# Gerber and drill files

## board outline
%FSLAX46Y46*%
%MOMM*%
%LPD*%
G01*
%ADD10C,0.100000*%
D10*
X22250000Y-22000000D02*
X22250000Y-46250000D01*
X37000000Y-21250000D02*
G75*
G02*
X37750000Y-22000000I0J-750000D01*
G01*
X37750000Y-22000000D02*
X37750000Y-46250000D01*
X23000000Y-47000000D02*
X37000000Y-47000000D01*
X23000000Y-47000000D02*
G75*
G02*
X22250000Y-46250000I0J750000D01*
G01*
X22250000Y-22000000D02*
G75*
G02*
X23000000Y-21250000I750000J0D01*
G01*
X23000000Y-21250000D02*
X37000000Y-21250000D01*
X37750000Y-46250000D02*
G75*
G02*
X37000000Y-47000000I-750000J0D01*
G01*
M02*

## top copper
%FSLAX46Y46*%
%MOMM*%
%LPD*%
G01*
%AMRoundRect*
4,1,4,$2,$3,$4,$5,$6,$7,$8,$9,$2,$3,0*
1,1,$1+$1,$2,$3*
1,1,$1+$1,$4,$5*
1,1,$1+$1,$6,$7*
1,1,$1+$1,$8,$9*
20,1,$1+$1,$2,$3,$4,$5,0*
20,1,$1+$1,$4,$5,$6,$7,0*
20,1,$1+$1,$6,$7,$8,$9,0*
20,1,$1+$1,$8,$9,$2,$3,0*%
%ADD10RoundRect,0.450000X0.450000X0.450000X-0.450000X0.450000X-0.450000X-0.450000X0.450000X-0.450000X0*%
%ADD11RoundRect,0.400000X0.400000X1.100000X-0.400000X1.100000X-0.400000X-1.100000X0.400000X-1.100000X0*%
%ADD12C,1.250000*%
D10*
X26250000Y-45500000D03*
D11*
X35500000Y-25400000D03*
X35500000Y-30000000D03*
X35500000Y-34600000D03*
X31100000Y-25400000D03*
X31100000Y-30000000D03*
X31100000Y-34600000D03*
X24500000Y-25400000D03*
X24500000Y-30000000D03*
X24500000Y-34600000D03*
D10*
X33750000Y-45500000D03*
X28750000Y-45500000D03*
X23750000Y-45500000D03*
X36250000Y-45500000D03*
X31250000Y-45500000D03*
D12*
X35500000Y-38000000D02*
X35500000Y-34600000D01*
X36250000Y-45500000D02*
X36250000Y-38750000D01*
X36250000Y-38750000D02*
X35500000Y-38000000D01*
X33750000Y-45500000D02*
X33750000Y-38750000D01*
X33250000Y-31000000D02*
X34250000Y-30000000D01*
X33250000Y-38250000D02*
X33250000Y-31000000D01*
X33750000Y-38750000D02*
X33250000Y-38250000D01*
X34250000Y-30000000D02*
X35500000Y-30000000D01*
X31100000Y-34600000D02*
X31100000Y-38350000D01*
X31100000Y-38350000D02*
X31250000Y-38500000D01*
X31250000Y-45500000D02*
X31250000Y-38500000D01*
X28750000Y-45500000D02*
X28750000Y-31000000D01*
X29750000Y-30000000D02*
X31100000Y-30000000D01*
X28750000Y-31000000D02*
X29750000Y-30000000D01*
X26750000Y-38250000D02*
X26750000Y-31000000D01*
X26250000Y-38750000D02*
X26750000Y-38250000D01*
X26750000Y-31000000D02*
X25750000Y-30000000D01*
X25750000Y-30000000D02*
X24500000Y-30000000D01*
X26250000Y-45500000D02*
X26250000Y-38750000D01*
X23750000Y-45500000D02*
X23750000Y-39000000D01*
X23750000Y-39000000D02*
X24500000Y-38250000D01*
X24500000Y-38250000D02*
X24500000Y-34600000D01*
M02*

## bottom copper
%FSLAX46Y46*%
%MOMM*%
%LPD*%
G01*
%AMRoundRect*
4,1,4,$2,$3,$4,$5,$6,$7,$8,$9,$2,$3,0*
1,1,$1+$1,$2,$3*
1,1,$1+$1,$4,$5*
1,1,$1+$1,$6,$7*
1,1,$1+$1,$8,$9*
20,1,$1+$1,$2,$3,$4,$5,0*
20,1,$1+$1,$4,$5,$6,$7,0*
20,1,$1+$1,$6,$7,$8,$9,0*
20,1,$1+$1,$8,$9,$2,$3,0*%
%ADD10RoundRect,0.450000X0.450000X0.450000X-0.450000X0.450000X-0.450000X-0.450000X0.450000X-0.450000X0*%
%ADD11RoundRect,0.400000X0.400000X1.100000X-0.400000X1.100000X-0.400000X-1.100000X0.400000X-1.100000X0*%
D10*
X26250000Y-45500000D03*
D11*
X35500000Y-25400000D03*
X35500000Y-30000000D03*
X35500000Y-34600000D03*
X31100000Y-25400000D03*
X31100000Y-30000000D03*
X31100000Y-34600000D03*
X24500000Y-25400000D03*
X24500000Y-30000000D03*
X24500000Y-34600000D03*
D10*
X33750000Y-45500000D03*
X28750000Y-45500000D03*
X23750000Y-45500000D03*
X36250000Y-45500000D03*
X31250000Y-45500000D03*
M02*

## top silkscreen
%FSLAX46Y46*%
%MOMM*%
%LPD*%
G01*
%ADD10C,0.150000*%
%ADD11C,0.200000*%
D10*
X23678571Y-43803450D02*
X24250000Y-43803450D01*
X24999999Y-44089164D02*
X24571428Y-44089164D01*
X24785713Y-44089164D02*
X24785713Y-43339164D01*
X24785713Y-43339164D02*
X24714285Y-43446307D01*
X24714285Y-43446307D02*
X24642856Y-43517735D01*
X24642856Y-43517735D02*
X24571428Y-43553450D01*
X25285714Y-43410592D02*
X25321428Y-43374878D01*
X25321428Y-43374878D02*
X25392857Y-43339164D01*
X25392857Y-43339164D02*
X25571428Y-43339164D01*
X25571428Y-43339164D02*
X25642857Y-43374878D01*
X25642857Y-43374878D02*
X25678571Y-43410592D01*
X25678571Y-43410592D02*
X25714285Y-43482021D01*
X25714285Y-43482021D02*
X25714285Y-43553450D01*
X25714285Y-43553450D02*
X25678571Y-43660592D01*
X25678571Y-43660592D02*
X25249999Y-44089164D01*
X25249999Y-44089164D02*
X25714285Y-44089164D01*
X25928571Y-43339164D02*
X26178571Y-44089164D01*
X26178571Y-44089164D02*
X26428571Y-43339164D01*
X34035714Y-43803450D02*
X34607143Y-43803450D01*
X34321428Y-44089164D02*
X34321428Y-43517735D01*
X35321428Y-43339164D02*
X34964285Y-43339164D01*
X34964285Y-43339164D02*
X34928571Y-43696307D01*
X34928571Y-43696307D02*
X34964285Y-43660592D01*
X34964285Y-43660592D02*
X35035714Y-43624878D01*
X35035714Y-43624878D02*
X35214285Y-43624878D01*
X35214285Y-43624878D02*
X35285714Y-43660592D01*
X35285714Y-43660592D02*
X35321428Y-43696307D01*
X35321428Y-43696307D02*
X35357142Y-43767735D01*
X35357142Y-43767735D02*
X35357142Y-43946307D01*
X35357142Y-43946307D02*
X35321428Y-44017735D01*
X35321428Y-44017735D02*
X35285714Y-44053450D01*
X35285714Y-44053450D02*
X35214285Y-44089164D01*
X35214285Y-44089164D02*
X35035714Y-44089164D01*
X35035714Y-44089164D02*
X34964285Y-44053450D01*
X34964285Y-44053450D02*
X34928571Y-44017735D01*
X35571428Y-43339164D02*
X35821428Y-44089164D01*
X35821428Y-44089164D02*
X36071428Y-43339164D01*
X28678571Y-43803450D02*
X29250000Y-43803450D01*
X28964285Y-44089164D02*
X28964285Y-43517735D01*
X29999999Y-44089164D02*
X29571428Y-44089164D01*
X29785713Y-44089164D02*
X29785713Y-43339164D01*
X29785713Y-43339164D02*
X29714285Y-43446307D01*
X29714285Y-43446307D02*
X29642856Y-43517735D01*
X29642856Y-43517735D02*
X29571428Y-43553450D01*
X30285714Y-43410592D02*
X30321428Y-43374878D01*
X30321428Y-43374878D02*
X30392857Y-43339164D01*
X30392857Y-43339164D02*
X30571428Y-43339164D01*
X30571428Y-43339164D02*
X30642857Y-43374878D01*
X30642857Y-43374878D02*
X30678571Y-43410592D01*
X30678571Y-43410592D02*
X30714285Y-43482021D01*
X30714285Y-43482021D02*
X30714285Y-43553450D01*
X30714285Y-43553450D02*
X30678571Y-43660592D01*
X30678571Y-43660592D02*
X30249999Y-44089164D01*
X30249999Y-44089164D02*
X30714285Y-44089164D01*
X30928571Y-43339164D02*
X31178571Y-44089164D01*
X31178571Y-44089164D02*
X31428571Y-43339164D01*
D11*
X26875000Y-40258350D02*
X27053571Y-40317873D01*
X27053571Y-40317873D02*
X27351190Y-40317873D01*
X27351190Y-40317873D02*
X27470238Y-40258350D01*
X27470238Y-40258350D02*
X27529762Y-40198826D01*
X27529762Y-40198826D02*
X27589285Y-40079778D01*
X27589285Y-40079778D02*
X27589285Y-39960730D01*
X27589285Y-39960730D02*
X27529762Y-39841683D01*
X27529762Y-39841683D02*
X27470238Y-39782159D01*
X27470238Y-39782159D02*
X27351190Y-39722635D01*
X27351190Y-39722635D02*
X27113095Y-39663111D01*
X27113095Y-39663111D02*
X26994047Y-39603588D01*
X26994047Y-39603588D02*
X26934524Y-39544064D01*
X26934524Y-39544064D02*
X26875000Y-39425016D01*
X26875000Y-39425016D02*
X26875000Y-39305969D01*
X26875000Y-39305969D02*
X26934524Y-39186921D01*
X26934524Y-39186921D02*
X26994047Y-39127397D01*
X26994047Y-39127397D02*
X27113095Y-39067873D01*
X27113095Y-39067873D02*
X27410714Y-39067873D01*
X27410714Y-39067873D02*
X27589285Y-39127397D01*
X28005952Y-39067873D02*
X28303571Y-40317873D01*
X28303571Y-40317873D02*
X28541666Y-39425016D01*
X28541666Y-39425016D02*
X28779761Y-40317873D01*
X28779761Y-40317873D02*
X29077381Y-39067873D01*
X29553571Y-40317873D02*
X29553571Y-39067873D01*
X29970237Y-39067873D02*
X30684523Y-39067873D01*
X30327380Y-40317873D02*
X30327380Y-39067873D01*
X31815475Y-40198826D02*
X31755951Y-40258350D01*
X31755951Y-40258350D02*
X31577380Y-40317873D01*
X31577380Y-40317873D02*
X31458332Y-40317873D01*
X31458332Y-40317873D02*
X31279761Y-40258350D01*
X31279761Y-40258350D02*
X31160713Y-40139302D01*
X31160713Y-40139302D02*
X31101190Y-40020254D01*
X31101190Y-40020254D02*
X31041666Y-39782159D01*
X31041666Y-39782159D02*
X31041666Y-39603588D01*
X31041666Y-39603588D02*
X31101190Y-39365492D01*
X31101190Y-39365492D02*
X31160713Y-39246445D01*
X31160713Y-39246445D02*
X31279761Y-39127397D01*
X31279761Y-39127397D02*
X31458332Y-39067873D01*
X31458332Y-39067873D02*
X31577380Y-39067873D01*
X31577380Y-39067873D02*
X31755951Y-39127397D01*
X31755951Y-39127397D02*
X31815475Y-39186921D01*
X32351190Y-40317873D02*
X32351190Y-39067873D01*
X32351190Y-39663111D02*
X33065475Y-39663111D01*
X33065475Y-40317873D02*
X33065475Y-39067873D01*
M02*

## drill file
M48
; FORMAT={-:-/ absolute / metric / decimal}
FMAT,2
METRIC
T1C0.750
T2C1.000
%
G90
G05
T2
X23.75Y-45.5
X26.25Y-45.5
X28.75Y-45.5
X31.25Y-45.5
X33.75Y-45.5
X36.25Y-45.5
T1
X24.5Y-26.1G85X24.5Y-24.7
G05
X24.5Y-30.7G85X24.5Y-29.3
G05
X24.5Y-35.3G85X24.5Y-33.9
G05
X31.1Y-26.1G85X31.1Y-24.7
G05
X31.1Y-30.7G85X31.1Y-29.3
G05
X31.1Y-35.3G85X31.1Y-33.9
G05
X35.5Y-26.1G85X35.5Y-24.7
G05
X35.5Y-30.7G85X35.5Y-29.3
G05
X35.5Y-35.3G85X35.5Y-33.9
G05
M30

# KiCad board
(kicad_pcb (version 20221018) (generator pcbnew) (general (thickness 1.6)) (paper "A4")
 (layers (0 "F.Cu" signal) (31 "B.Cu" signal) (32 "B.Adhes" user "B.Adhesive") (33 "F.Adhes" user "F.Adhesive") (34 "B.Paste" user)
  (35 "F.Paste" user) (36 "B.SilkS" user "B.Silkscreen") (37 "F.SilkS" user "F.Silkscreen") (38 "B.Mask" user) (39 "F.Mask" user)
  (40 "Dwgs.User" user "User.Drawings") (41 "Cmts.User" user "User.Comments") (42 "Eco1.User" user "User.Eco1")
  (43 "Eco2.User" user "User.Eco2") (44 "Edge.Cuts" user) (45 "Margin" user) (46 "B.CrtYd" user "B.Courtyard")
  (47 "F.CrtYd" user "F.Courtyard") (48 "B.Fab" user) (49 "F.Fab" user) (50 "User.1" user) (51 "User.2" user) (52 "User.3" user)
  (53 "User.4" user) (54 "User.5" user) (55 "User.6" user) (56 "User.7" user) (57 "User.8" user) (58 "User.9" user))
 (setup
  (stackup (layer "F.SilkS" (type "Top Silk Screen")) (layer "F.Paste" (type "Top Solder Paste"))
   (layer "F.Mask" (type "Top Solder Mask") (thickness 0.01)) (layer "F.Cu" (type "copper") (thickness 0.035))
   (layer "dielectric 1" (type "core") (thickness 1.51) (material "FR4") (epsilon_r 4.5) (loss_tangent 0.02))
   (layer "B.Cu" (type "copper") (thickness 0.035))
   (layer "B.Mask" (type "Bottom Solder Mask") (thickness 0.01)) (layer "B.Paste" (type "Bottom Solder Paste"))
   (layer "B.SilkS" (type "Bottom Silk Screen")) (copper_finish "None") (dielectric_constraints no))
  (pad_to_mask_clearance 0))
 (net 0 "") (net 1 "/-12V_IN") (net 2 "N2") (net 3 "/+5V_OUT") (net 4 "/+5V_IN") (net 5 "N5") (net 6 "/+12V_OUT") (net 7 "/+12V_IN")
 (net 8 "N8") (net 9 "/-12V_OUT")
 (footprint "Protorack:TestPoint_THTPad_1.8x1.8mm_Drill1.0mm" (layer "B.Cu") (at 26.25 45.5 180)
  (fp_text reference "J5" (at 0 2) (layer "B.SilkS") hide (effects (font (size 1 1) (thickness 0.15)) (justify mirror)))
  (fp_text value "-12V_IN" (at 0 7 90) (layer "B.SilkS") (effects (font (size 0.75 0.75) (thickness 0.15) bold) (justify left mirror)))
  (pad "1" thru_hole roundrect (at 0 0 180) (size 1.8 1.8) (drill 1) (layers "*.Cu" "*.Mask") (roundrect_rratio 0.25) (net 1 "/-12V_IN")))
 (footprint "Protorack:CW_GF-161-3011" (layer "B.Cu") (at 30 30 180)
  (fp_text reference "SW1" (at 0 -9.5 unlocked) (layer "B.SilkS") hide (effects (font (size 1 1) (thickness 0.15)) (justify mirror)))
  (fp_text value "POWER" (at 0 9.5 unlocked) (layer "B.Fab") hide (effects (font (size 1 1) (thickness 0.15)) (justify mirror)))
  (pad "1" thru_hole roundrect (at -5.5 4.6 180) (size 1.6 3) (drill oval 0.75 2.15) (layers "*.Cu" "*.Mask") (roundrect_rratio 0.25)
   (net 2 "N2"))
  (pad "2" thru_hole roundrect (at -5.5 0 180) (size 1.6 3) (drill oval 0.75 2.15) (layers "*.Cu" "*.Mask") (roundrect_rratio 0.25)
   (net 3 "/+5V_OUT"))
  (pad "3" thru_hole roundrect (at -5.5 -4.6 180) (size 1.6 3) (drill oval 0.75 2.15) (layers "*.Cu" "*.Mask") (roundrect_rratio 0.25)
   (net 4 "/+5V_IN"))
  (pad "4" thru_hole roundrect (at -1.1 4.6 180) (size 1.6 3) (drill oval 0.75 2.15) (layers "*.Cu" "*.Mask") (roundrect_rratio 0.25)
   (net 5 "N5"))
  (pad "5" thru_hole roundrect (at -1.1 0 180) (size 1.6 3) (drill oval 0.75 2.15) (layers "*.Cu" "*.Mask") (roundrect_rratio 0.25)
   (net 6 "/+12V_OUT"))
  (pad "6" thru_hole roundrect (at -1.1 -4.6 180) (size 1.6 3) (drill oval 0.75 2.15) (layers "*.Cu" "*.Mask") (roundrect_rratio 0.25)
   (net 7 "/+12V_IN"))
  (pad "7" thru_hole roundrect (at 5.5 4.6 180) (size 1.6 3) (drill oval 0.75 2.15) (layers "*.Cu" "*.Mask") (roundrect_rratio 0.25)
   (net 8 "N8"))
  (pad "8" thru_hole roundrect (at 5.5 0 180) (size 1.6 3) (drill oval 0.75 2.15) (layers "*.Cu" "*.Mask") (roundrect_rratio 0.25)
   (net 1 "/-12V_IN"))
  (pad "9" thru_hole roundrect (at 5.5 -4.6 180) (size 1.6 3) (drill oval 0.75 2.15) (layers "*.Cu" "*.Mask") (roundrect_rratio 0.25)
   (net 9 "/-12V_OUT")))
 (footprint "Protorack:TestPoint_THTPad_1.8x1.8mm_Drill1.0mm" (layer "B.Cu") (at 33.75 45.5 180)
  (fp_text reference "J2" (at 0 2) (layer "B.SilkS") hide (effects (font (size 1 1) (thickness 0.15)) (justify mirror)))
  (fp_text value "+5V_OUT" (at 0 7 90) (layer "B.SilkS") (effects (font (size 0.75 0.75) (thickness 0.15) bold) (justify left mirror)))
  (pad "1" thru_hole roundrect (at 0 0 180) (size 1.8 1.8) (drill 1) (layers "*.Cu" "*.Mask") (roundrect_rratio 0.25) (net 3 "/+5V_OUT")))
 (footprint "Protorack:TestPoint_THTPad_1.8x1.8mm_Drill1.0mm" (layer "B.Cu") (at 28.75 45.5 180)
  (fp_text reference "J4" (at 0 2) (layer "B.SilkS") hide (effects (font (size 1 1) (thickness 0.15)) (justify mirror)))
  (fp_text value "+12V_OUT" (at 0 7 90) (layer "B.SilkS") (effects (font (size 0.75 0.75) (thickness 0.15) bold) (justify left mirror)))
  (pad "1" thru_hole roundrect (at 0 0 180) (size 1.8 1.8) (drill 1) (layers "*.Cu" "*.Mask") (roundrect_rratio 0.25) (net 6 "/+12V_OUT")))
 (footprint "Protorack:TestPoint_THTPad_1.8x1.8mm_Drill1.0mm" (layer "B.Cu") (at 23.75 45.5 180)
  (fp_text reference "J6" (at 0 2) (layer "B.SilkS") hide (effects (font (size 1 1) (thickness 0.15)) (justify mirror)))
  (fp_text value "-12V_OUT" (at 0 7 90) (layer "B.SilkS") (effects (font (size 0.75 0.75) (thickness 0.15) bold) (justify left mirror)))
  (pad "1" thru_hole roundrect (at 0 0 180) (size 1.8 1.8) (drill 1) (layers "*.Cu" "*.Mask") (roundrect_rratio 0.25) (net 9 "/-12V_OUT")))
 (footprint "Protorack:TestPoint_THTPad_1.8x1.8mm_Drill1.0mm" (layer "B.Cu") (at 36.25 45.5 180)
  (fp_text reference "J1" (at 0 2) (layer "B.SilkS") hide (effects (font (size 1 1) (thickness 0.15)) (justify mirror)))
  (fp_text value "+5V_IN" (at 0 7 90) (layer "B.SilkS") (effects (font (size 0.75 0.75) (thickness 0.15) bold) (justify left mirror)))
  (pad "1" thru_hole roundrect (at 0 0 180) (size 1.8 1.8) (drill 1) (layers "*.Cu" "*.Mask") (roundrect_rratio 0.25) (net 4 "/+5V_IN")))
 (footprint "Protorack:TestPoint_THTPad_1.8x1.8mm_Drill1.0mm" (layer "B.Cu") (at 31.25 45.5 180)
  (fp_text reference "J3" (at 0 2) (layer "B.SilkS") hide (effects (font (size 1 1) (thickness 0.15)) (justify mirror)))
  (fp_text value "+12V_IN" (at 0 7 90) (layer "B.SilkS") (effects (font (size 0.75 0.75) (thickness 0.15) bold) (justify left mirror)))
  (pad "1" thru_hole roundrect (at 0 0 180) (size 1.8 1.8) (drill 1) (layers "*.Cu" "*.Mask") (roundrect_rratio 0.25) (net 7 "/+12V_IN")))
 (gr_line (start 22.25 22) (end 22.25 46.25) (stroke (width 0.1) (type solid)) (layer "Edge.Cuts"))
 (gr_arc (start 37 21.25) (mid 37.53033 21.46967) (end 37.75 22) (stroke (width 0.1) (type solid)) (layer "Edge.Cuts"))
 (gr_line (start 37.75 22) (end 37.75 46.25) (stroke (width 0.1) (type solid)) (layer "Edge.Cuts"))
 (gr_line (start 23 47) (end 37 47) (stroke (width 0.1) (type solid)) (layer "Edge.Cuts"))
 (gr_arc (start 23 47) (mid 22.46967 46.78033) (end 22.25 46.25) (stroke (width 0.1) (type solid)) (layer "Edge.Cuts"))
 (gr_arc (start 22.25 22) (mid 22.46967 21.46967) (end 23 21.25) (stroke (width 0.1) (type solid)) (layer "Edge.Cuts"))
 (gr_line (start 23 21.25) (end 37 21.25) (stroke (width 0.1) (type solid)) (layer "Edge.Cuts"))
 (gr_arc (start 37.75 46.25) (mid 37.53033 46.78033) (end 37 47) (stroke (width 0.1) (type solid)) (layer "Edge.Cuts"))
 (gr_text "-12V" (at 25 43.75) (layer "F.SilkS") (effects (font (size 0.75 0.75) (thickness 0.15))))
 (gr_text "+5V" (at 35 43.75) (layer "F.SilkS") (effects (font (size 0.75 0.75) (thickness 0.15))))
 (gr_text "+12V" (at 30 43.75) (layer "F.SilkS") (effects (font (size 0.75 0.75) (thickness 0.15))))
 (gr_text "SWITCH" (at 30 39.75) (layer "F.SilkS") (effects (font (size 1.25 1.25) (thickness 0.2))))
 (segment (start 35.5 38) (end 35.5 34.6) (width 1.25) (layer "F.Cu") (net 4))
 (segment (start 36.25 45.5) (end 36.25 38.75) (width 1.25) (layer "F.Cu") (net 4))
 (segment (start 36.25 38.75) (end 35.5 38) (width 1.25) (layer "F.Cu") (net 4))
 (segment (start 33.75 45.5) (end 33.75 38.75) (width 1.25) (layer "F.Cu") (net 3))
 (segment (start 33.25 31) (end 34.25 30) (width 1.25) (layer "F.Cu") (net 3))
 (segment (start 33.25 38.25) (end 33.25 31) (width 1.25) (layer "F.Cu") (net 3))
 (segment (start 33.75 38.75) (end 33.25 38.25) (width 1.25) (layer "F.Cu") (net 3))
 (segment (start 34.25 30) (end 35.5 30) (width 1.25) (layer "F.Cu") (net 3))
 (segment (start 31.1 34.6) (end 31.1 38.35) (width 1.25) (layer "F.Cu") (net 7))
 (segment (start 31.1 38.35) (end 31.25 38.5) (width 1.25) (layer "F.Cu") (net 7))
 (segment (start 31.25 45.5) (end 31.25 38.5) (width 1.25) (layer "F.Cu") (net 7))
 (segment (start 28.75 45.5) (end 28.75 31) (width 1.25) (layer "F.Cu") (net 6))
 (segment (start 29.75 30) (end 31.1 30) (width 1.25) (layer "F.Cu") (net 6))
 (segment (start 28.75 31) (end 29.75 30) (width 1.25) (layer "F.Cu") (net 6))
 (segment (start 26.75 38.25) (end 26.75 31) (width 1.25) (layer "F.Cu") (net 1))
 (segment (start 26.25 38.75) (end 26.75 38.25) (width 1.25) (layer "F.Cu") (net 1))
 (segment (start 26.75 31) (end 25.75 30) (width 1.25) (layer "F.Cu") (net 1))
 (segment (start 25.75 30) (end 24.5 30) (width 1.25) (layer "F.Cu") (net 1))
 (segment (start 26.25 45.5) (end 26.25 38.75) (width 1.25) (layer "F.Cu") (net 1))
 (segment (start 23.75 45.5) (end 23.75 39) (width 1.25) (layer "F.Cu") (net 9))
 (segment (start 23.75 39) (end 24.5 38.25) (width 1.25) (layer "F.Cu") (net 9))
 (segment (start 24.5 38.25) (end 24.5 34.6) (width 1.25) (layer "F.Cu") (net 9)))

